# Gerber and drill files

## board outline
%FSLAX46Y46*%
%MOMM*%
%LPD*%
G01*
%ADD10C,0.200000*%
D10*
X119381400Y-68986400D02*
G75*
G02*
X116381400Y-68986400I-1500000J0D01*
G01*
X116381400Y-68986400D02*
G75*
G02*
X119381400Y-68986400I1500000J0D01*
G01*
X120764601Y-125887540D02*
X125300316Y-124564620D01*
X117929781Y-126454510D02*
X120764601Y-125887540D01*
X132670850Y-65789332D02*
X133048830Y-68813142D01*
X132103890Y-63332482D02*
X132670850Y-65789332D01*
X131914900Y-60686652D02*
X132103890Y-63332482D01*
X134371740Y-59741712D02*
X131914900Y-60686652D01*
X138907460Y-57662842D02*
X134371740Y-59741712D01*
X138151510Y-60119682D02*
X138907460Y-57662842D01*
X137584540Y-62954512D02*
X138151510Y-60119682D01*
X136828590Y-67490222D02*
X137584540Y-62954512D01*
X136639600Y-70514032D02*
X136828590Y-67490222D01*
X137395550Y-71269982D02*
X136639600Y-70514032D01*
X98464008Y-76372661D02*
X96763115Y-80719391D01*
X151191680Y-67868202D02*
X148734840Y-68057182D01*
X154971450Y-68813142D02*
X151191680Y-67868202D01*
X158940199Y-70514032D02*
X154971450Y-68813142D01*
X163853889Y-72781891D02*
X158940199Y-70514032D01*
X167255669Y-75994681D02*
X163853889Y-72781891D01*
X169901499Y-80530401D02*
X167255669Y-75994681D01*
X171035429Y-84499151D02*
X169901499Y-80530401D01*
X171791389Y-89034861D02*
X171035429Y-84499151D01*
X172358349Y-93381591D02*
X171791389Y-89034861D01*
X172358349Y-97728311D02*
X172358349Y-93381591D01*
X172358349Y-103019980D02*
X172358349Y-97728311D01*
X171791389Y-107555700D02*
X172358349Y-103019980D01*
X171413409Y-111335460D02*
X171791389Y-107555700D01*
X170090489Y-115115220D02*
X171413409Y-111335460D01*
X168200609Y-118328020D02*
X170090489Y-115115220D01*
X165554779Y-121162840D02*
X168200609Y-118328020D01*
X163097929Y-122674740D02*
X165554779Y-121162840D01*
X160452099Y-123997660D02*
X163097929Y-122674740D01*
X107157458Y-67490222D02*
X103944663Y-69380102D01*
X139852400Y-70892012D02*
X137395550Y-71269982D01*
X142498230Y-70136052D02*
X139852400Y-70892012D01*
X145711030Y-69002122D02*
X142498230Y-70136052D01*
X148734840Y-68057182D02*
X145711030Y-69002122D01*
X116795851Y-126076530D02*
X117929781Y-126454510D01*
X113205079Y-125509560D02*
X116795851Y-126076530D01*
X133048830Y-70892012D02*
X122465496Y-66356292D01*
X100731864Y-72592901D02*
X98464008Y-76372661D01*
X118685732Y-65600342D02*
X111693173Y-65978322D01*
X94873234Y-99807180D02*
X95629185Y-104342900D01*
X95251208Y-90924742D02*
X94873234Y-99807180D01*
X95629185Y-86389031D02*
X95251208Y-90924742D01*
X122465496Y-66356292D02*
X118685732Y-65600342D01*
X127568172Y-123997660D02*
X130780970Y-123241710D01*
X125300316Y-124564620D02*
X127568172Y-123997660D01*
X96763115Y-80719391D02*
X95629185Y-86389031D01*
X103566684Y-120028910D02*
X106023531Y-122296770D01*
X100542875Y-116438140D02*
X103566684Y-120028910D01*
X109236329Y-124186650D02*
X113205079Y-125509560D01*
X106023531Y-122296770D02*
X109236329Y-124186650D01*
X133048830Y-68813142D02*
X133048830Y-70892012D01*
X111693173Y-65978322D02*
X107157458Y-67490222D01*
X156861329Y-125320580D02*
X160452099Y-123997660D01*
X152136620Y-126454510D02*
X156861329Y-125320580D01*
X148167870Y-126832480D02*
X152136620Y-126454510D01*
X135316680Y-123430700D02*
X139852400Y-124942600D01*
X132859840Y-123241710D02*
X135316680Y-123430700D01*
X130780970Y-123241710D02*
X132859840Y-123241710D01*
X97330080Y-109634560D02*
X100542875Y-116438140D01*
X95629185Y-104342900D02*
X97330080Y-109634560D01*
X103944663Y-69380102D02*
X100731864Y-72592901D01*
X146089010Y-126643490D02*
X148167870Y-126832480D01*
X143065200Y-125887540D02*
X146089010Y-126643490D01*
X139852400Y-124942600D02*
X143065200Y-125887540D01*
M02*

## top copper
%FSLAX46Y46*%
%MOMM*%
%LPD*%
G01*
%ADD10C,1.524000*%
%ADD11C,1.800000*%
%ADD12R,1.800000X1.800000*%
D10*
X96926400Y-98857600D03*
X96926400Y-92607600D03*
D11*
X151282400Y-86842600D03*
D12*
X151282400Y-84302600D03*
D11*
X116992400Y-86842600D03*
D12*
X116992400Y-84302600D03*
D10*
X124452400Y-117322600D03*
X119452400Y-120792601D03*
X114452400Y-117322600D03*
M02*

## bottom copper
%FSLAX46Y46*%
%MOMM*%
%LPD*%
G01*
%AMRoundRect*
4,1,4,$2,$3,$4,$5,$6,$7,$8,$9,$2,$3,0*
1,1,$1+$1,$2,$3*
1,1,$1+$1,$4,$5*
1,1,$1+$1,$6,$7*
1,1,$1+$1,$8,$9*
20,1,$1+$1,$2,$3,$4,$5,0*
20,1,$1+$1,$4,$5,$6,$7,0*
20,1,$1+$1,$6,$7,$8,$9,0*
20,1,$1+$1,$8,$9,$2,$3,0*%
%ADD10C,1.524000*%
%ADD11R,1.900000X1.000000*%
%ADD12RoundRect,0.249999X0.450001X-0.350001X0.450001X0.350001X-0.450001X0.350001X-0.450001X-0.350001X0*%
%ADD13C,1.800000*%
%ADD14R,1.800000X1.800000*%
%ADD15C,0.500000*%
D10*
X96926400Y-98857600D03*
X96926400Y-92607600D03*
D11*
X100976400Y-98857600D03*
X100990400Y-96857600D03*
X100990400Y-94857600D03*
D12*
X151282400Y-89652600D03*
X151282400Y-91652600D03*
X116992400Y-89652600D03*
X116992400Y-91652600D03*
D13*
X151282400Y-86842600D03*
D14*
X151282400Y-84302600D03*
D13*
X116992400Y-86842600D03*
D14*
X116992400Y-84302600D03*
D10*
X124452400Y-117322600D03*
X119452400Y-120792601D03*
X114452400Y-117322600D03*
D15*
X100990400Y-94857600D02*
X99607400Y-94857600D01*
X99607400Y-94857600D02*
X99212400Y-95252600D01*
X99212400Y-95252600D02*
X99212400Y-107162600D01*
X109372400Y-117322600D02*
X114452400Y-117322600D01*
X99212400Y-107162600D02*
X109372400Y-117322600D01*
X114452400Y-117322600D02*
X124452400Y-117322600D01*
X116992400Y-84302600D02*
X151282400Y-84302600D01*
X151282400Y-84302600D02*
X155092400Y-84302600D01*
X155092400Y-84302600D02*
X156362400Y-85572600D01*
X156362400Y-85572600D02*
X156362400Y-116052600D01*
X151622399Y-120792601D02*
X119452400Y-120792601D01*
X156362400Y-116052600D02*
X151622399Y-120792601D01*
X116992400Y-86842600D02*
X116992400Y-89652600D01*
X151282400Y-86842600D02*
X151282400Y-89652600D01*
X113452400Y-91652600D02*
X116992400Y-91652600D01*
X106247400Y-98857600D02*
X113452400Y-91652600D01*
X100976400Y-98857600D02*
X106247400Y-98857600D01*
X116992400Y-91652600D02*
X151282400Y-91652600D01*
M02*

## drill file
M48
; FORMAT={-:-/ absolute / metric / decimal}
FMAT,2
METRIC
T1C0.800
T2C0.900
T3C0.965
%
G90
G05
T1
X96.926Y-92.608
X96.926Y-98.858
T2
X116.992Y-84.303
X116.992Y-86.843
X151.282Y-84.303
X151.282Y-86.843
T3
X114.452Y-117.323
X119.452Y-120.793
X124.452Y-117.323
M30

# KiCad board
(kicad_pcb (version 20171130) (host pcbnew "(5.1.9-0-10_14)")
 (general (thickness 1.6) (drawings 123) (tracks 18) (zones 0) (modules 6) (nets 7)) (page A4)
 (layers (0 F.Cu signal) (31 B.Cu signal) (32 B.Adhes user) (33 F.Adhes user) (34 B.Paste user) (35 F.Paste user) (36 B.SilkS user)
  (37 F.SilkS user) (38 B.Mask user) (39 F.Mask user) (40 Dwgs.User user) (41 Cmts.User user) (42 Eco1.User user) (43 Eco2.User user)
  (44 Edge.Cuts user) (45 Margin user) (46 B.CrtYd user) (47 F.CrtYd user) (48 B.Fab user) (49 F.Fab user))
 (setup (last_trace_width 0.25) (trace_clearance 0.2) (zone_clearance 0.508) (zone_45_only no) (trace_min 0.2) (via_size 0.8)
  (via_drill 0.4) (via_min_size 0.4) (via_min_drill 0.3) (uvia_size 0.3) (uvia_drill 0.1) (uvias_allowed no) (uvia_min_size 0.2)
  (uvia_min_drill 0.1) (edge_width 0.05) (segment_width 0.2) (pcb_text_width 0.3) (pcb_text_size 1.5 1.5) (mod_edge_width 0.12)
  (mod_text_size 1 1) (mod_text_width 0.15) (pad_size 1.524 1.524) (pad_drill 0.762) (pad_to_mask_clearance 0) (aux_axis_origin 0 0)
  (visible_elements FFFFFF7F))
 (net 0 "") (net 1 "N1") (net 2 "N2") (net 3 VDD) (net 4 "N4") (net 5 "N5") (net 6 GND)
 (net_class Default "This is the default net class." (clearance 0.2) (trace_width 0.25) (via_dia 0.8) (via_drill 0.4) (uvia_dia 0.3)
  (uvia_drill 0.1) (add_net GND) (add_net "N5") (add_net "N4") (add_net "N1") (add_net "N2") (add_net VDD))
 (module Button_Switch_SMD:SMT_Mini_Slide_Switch (layer B.Cu) (at 99.2124 95.7326 90)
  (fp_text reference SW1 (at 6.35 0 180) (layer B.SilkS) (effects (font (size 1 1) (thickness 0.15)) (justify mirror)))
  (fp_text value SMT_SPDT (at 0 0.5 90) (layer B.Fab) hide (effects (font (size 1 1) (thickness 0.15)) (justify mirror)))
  (pad "" thru_hole circle (at -3.125 -2.286 90) (size 1.524 1.524) (drill 0.8) (layers *.Cu *.Mask))
  (pad "" thru_hole circle (at 3.125 -2.286 90) (size 1.524 1.524) (drill 0.8) (layers *.Cu *.Mask))
  (pad 1 smd rect (at -3.125 1.764 90) (size 1 1.9) (layers B.Cu B.Paste B.Mask) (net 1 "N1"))
  (pad 2 smd rect (at -1.125 1.778 90) (size 1 1.9) (layers B.Cu B.Paste B.Mask) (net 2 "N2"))
  (pad 3 smd rect (at 0.875 1.778 90) (size 1 1.9) (layers B.Cu B.Paste B.Mask) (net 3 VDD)))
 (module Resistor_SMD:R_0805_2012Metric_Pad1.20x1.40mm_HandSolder (layer B.Cu) (at 151.2824 90.6526 90)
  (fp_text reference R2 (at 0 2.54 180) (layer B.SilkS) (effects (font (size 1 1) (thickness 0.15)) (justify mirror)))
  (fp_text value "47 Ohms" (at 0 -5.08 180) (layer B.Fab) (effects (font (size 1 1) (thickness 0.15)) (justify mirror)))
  (pad 2 smd roundrect (at 1 0 90) (size 1.2 1.4) (layers B.Cu B.Paste B.Mask) (roundrect_rratio 0.2083325) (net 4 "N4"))
  (pad 1 smd roundrect (at -1 0 90) (size 1.2 1.4) (layers B.Cu B.Paste B.Mask) (roundrect_rratio 0.2083325) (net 1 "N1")))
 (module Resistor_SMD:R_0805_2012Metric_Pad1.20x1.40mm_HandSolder (layer B.Cu) (at 116.9924 90.6526 90)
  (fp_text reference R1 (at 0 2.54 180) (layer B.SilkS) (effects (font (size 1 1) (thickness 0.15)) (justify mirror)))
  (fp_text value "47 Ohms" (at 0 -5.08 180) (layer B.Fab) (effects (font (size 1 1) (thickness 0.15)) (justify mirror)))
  (pad 2 smd roundrect (at 1 0 90) (size 1.2 1.4) (layers B.Cu B.Paste B.Mask) (roundrect_rratio 0.2083325) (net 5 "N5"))
  (pad 1 smd roundrect (at -1 0 90) (size 1.2 1.4) (layers B.Cu B.Paste B.Mask) (roundrect_rratio 0.2083325) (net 1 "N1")))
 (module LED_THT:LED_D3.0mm (layer F.Cu) (at 151.2824 84.3026 270)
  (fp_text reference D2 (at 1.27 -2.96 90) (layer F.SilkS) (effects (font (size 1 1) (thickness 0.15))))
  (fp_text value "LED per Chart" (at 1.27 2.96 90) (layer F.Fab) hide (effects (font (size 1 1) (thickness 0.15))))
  (pad 2 thru_hole circle (at 2.54 0 270) (size 1.8 1.8) (drill 0.9) (layers *.Cu *.Mask) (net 4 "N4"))
  (pad 1 thru_hole rect (at 0 0 270) (size 1.8 1.8) (drill 0.9) (layers *.Cu *.Mask) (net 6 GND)))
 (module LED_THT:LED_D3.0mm (layer F.Cu) (at 116.9924 84.3026 270)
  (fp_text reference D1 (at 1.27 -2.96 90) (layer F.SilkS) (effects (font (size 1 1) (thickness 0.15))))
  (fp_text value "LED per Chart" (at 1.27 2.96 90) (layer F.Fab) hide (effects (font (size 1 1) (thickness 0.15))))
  (pad 2 thru_hole circle (at 2.54 0 270) (size 1.8 1.8) (drill 0.9) (layers *.Cu *.Mask) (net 5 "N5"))
  (pad 1 thru_hole rect (at 0 0 270) (size 1.8 1.8) (drill 0.9) (layers *.Cu *.Mask) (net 6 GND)))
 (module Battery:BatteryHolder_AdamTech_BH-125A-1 (layer B.Cu) (at 114.4524 117.3226)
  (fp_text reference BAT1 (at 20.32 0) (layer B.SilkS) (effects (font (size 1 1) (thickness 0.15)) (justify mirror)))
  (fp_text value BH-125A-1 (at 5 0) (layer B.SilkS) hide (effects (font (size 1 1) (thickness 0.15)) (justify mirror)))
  (pad POS2 thru_hole circle (at 10 0) (size 1.524 1.524) (drill 0.9652) (layers *.Cu *.Mask) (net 3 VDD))
  (pad NEG thru_hole circle (at 5 3.470001) (size 1.524 1.524) (drill 0.9652) (layers *.Cu *.Mask) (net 6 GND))
  (pad POS1 thru_hole circle (at 0 0) (size 1.524 1.524) (drill 0.9652) (layers *.Cu *.Mask) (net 3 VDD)))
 (gr_circle (center 117.8814 68.9864) (end 119.3814 68.9864) (layer Edge.Cuts) (width 0.2))
 (gr_line (start 120.764601 125.88754) (end 125.300316 124.56462) (layer Edge.Cuts) (width 0.2))
 (gr_line (start 117.929781 126.45451) (end 120.764601 125.88754) (layer Edge.Cuts) (width 0.2))
 (gr_line (start 132.67085 65.789332) (end 133.04883 68.813142) (layer Edge.Cuts) (width 0.2))
 (gr_line (start 132.10389 63.332482) (end 132.67085 65.789332) (layer Edge.Cuts) (width 0.2))
 (gr_line (start 131.9149 60.686652) (end 132.10389 63.332482) (layer Edge.Cuts) (width 0.2))
 (gr_line (start 134.37174 59.741712) (end 131.9149 60.686652) (layer Edge.Cuts) (width 0.2))
 (gr_line (start 138.90746 57.662842) (end 134.37174 59.741712) (layer Edge.Cuts) (width 0.2))
 (gr_line (start 138.15151 60.119682) (end 138.90746 57.662842) (layer Edge.Cuts) (width 0.2))
 (gr_line (start 137.58454 62.954512) (end 138.15151 60.119682) (layer Edge.Cuts) (width 0.2))
 (gr_line (start 136.82859 67.490222) (end 137.58454 62.954512) (layer Edge.Cuts) (width 0.2))
 (gr_line (start 136.6396 70.514032) (end 136.82859 67.490222) (layer Edge.Cuts) (width 0.2))
 (gr_line (start 137.39555 71.269982) (end 136.6396 70.514032) (layer Edge.Cuts) (width 0.2))
 (gr_line (start 98.464008 76.372661) (end 96.763115 80.719391) (layer Edge.Cuts) (width 0.2))
 (gr_line (start 151.19168 67.868202) (end 148.73484 68.057182) (layer Edge.Cuts) (width 0.2))
 (gr_line (start 154.97145 68.813142) (end 151.19168 67.868202) (layer Edge.Cuts) (width 0.2))
 (gr_line (start 158.940199 70.514032) (end 154.97145 68.813142) (layer Edge.Cuts) (width 0.2))
 (gr_line (start 163.853889 72.781891) (end 158.940199 70.514032) (layer Edge.Cuts) (width 0.2))
 (gr_line (start 167.255669 75.994681) (end 163.853889 72.781891) (layer Edge.Cuts) (width 0.2))
 (gr_line (start 169.901499 80.530401) (end 167.255669 75.994681) (layer Edge.Cuts) (width 0.2))
 (gr_line (start 171.035429 84.499151) (end 169.901499 80.530401) (layer Edge.Cuts) (width 0.2))
 (gr_line (start 171.791389 89.034861) (end 171.035429 84.499151) (layer Edge.Cuts) (width 0.2))
 (gr_line (start 172.358349 93.381591) (end 171.791389 89.034861) (layer Edge.Cuts) (width 0.2))
 (gr_line (start 172.358349 97.728311) (end 172.358349 93.381591) (layer Edge.Cuts) (width 0.2))
 (gr_line (start 172.358349 103.01998) (end 172.358349 97.728311) (layer Edge.Cuts) (width 0.2))
 (gr_line (start 171.791389 107.5557) (end 172.358349 103.01998) (layer Edge.Cuts) (width 0.2))
 (gr_line (start 171.413409 111.33546) (end 171.791389 107.5557) (layer Edge.Cuts) (width 0.2))
 (gr_line (start 170.090489 115.11522) (end 171.413409 111.33546) (layer Edge.Cuts) (width 0.2))
 (gr_line (start 168.200609 118.32802) (end 170.090489 115.11522) (layer Edge.Cuts) (width 0.2))
 (gr_line (start 165.554779 121.16284) (end 168.200609 118.32802) (layer Edge.Cuts) (width 0.2))
 (gr_line (start 163.097929 122.67474) (end 165.554779 121.16284) (layer Edge.Cuts) (width 0.2))
 (gr_line (start 160.452099 123.99766) (end 163.097929 122.67474) (layer Edge.Cuts) (width 0.2))
 (gr_line (start 107.157458 67.490222) (end 103.944663 69.380102) (layer Edge.Cuts) (width 0.2))
 (gr_line (start 139.8524 70.892012) (end 137.39555 71.269982) (layer Edge.Cuts) (width 0.2))
 (gr_line (start 142.49823 70.136052) (end 139.8524 70.892012) (layer Edge.Cuts) (width 0.2))
 (gr_line (start 145.71103 69.002122) (end 142.49823 70.136052) (layer Edge.Cuts) (width 0.2))
 (gr_line (start 148.73484 68.057182) (end 145.71103 69.002122) (layer Edge.Cuts) (width 0.2))
 (gr_line (start 116.795851 126.07653) (end 117.929781 126.45451) (layer Edge.Cuts) (width 0.2))
 (gr_line (start 113.205079 125.50956) (end 116.795851 126.07653) (layer Edge.Cuts) (width 0.2))
 (gr_line (start 133.04883 70.892012) (end 122.465496 66.356292) (layer Edge.Cuts) (width 0.2))
 (gr_line (start 100.731864 72.592901) (end 98.464008 76.372661) (layer Edge.Cuts) (width 0.2))
 (gr_line (start 118.685732 65.600342) (end 111.693173 65.978322) (layer Edge.Cuts) (width 0.2))
 (gr_line (start 94.873234 99.80718) (end 95.629185 104.3429) (layer Edge.Cuts) (width 0.2))
 (gr_line (start 95.251208 90.924742) (end 94.873234 99.80718) (layer Edge.Cuts) (width 0.2))
 (gr_line (start 95.629185 86.389031) (end 95.251208 90.924742) (layer Edge.Cuts) (width 0.2))
 (gr_line (start 122.465496 66.356292) (end 118.685732 65.600342) (layer Edge.Cuts) (width 0.2))
 (gr_line (start 127.568172 123.99766) (end 130.78097 123.24171) (layer Edge.Cuts) (width 0.2))
 (gr_line (start 125.300316 124.56462) (end 127.568172 123.99766) (layer Edge.Cuts) (width 0.2))
 (gr_line (start 96.763115 80.719391) (end 95.629185 86.389031) (layer Edge.Cuts) (width 0.2))
 (gr_line (start 103.566684 120.02891) (end 106.023531 122.29677) (layer Edge.Cuts) (width 0.2))
 (gr_line (start 100.542875 116.43814) (end 103.566684 120.02891) (layer Edge.Cuts) (width 0.2))
 (gr_line (start 109.236329 124.18665) (end 113.205079 125.50956) (layer Edge.Cuts) (width 0.2))
 (gr_line (start 106.023531 122.29677) (end 109.236329 124.18665) (layer Edge.Cuts) (width 0.2))
 (gr_line (start 133.04883 68.813142) (end 133.04883 70.892012) (layer Edge.Cuts) (width 0.2))
 (gr_line (start 111.693173 65.978322) (end 107.157458 67.490222) (layer Edge.Cuts) (width 0.2))
 (gr_line (start 156.861329 125.32058) (end 160.452099 123.99766) (layer Edge.Cuts) (width 0.2))
 (gr_line (start 152.13662 126.45451) (end 156.861329 125.32058) (layer Edge.Cuts) (width 0.2))
 (gr_line (start 148.16787 126.83248) (end 152.13662 126.45451) (layer Edge.Cuts) (width 0.2))
 (gr_line (start 135.31668 123.4307) (end 139.8524 124.9426) (layer Edge.Cuts) (width 0.2))
 (gr_line (start 132.85984 123.24171) (end 135.31668 123.4307) (layer Edge.Cuts) (width 0.2))
 (gr_line (start 130.78097 123.24171) (end 132.85984 123.24171) (layer Edge.Cuts) (width 0.2))
 (gr_line (start 97.33008 109.63456) (end 100.542875 116.43814) (layer Edge.Cuts) (width 0.2))
 (gr_line (start 95.629185 104.3429) (end 97.33008 109.63456) (layer Edge.Cuts) (width 0.2))
 (gr_line (start 103.944663 69.380102) (end 100.731864 72.592901) (layer Edge.Cuts) (width 0.2))
 (gr_line (start 146.08901 126.64349) (end 148.16787 126.83248) (layer Edge.Cuts) (width 0.2))
 (gr_line (start 143.0652 125.88754) (end 146.08901 126.64349) (layer Edge.Cuts) (width 0.2))
 (gr_line (start 139.8524 124.9426) (end 143.0652 125.88754) (layer Edge.Cuts) (width 0.2))
 (segment (start 100.9904 94.8576) (end 99.6074 94.8576) (width 0.5) (layer B.Cu) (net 3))
 (segment (start 99.6074 94.8576) (end 99.2124 95.2526) (width 0.5) (layer B.Cu) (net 3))
 (segment (start 99.2124 95.2526) (end 99.2124 107.1626) (width 0.5) (layer B.Cu) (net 3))
 (segment (start 109.3724 117.3226) (end 114.4524 117.3226) (width 0.5) (layer B.Cu) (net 3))
 (segment (start 99.2124 107.1626) (end 109.3724 117.3226) (width 0.5) (layer B.Cu) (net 3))
 (segment (start 114.4524 117.3226) (end 124.4524 117.3226) (width 0.5) (layer B.Cu) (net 3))
 (segment (start 116.9924 84.3026) (end 151.2824 84.3026) (width 0.5) (layer B.Cu) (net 6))
 (segment (start 151.2824 84.3026) (end 155.0924 84.3026) (width 0.5) (layer B.Cu) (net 6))
 (segment (start 155.0924 84.3026) (end 156.3624 85.5726) (width 0.5) (layer B.Cu) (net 6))
 (segment (start 156.3624 85.5726) (end 156.3624 116.0526) (width 0.5) (layer B.Cu) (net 6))
 (segment (start 151.622399 120.792601) (end 119.4524 120.792601) (width 0.5) (layer B.Cu) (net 6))
 (segment (start 156.3624 116.0526) (end 151.622399 120.792601) (width 0.5) (layer B.Cu) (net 6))
 (segment (start 116.9924 86.8426) (end 116.9924 89.6526) (width 0.5) (layer B.Cu) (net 5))
 (segment (start 151.2824 86.8426) (end 151.2824 89.6526) (width 0.5) (layer B.Cu) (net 4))
 (segment (start 113.4524 91.6526) (end 116.9924 91.6526) (width 0.5) (layer B.Cu) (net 1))
 (segment (start 106.2474 98.8576) (end 113.4524 91.6526) (width 0.5) (layer B.Cu) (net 1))
 (segment (start 100.9764 98.8576) (end 106.2474 98.8576) (width 0.5) (layer B.Cu) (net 1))
 (segment (start 116.9924 91.6526) (end 151.2824 91.6526) (width 0.5) (layer B.Cu) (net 1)))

